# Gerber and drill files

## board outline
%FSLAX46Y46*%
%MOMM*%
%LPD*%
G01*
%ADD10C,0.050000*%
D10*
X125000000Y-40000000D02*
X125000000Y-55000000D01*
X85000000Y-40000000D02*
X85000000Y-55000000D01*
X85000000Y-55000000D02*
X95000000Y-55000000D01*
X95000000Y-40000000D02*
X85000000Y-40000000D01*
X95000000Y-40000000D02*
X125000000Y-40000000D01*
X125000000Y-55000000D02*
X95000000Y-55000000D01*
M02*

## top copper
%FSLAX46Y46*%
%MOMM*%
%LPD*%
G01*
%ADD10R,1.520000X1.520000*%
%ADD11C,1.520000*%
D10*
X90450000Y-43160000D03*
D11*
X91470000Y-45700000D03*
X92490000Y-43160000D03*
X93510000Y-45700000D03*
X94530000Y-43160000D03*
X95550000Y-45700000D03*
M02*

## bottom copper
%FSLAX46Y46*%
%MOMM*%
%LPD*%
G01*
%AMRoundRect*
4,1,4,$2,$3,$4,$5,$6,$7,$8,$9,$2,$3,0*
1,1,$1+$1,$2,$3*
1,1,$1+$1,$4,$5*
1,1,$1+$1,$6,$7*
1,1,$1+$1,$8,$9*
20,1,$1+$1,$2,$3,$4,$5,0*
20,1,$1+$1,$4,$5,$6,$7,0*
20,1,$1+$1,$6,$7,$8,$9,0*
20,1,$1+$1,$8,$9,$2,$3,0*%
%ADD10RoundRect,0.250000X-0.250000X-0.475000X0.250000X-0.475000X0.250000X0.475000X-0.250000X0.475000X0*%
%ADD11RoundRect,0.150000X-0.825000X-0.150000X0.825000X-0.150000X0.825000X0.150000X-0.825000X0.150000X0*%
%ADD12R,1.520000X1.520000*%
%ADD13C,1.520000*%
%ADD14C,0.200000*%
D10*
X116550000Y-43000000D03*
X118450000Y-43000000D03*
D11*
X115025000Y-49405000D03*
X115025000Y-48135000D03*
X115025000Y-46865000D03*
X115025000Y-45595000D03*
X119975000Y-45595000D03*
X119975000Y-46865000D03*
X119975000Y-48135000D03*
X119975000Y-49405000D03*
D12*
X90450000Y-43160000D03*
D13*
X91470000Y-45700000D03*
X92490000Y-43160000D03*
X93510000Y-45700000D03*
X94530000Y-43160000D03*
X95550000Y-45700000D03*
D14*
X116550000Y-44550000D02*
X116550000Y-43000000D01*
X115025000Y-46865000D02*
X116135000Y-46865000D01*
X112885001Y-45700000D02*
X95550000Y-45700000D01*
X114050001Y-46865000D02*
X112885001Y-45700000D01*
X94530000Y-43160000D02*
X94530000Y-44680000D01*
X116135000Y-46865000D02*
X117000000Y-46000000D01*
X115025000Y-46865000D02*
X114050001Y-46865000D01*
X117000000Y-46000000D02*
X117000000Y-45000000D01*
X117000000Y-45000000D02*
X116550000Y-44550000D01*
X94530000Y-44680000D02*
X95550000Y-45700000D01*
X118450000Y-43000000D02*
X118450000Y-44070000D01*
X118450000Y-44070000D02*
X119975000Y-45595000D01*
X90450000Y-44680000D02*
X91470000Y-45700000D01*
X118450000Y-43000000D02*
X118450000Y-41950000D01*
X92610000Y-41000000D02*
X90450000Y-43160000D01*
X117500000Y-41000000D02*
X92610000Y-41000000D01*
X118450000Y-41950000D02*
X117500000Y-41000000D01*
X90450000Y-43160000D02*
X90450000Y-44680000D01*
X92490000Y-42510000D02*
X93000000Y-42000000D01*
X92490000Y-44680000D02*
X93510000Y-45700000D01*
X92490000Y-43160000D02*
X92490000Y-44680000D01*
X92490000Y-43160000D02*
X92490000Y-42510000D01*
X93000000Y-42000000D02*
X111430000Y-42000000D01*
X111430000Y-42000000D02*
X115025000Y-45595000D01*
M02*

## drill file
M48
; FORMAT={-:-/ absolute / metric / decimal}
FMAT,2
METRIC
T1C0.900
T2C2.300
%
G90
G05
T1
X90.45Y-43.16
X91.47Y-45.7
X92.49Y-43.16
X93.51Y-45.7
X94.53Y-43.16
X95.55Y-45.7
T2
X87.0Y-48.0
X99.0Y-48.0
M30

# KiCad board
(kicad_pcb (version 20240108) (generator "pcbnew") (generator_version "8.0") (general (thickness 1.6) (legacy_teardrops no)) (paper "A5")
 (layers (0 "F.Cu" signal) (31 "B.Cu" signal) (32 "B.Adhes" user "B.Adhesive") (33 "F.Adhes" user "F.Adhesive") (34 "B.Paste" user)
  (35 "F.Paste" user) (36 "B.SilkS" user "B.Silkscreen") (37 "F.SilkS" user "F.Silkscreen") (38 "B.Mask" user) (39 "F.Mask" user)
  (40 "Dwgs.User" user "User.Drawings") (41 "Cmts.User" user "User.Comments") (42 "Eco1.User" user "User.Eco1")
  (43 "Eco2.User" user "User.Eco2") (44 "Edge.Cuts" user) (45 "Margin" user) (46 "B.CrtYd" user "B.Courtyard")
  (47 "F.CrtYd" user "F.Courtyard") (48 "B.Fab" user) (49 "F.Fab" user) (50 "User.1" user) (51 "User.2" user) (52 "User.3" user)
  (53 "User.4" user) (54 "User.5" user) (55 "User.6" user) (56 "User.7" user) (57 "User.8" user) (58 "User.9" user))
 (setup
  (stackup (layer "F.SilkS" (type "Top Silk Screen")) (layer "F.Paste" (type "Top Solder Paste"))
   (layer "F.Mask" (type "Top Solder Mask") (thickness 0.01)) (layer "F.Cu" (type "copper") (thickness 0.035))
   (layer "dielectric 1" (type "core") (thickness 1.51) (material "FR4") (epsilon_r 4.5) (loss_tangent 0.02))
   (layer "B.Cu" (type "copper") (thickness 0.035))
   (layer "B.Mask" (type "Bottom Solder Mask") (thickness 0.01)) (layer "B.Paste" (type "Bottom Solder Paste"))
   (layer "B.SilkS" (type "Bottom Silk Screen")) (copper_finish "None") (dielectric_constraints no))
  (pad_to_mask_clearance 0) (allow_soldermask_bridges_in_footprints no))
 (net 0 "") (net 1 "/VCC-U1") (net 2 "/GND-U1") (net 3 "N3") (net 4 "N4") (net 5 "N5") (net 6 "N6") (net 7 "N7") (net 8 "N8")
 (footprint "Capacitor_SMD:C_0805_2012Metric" (layer "B.Cu") (at 117.5 43)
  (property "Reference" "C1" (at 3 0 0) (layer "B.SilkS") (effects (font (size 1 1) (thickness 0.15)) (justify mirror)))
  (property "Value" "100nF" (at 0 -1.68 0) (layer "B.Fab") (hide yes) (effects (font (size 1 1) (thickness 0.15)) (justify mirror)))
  (pad "1" smd roundrect (at -0.95 0) (size 1 1.45) (layers "B.Cu" "B.Paste" "B.Mask") (roundrect_rratio 0.25) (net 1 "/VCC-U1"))
  (pad "2" smd roundrect (at 0.95 0) (size 1 1.45) (layers "B.Cu" "B.Paste" "B.Mask") (roundrect_rratio 0.25) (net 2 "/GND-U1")))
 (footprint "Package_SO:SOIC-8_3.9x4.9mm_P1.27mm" (layer "B.Cu") (at 117.5 47.5)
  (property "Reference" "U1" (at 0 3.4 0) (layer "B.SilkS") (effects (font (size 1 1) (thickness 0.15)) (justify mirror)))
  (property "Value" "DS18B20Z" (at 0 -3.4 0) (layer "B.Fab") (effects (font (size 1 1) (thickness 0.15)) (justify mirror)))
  (pad "1" smd roundrect (at -2.475 1.905) (size 1.95 0.6) (layers "B.Cu" "B.Paste" "B.Mask") (roundrect_rratio 0.25) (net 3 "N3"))
  (pad "2" smd roundrect (at -2.475 0.635) (size 1.95 0.6) (layers "B.Cu" "B.Paste" "B.Mask") (roundrect_rratio 0.25) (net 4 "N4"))
  (pad "3" smd roundrect (at -2.475 -0.635) (size 1.95 0.6) (layers "B.Cu" "B.Paste" "B.Mask") (roundrect_rratio 0.25) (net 1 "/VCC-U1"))
  (pad "4" smd roundrect (at -2.475 -1.905) (size 1.95 0.6) (layers "B.Cu" "B.Paste" "B.Mask") (roundrect_rratio 0.25) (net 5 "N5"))
  (pad "5" smd roundrect (at 2.475 -1.905) (size 1.95 0.6) (layers "B.Cu" "B.Paste" "B.Mask") (roundrect_rratio 0.25) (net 2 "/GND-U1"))
  (pad "6" smd roundrect (at 2.475 -0.635) (size 1.95 0.6) (layers "B.Cu" "B.Paste" "B.Mask") (roundrect_rratio 0.25) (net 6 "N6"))
  (pad "7" smd roundrect (at 2.475 0.635) (size 1.95 0.6) (layers "B.Cu" "B.Paste" "B.Mask") (roundrect_rratio 0.25) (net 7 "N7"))
  (pad "8" smd roundrect (at 2.475 1.905) (size 1.95 0.6) (layers "B.Cu" "B.Paste" "B.Mask") (roundrect_rratio 0.25) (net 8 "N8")))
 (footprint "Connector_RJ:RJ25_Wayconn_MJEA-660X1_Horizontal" (layer "B.Cu") (at 90.45 43.16 180)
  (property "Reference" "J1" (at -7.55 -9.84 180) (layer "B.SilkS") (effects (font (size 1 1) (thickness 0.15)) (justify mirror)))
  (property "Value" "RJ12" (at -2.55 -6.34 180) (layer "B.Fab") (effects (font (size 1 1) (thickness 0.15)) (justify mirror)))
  (pad "" np_thru_hole circle (at -8.55 -4.84 180) (size 2.3 2.3) (drill 2.3) (layers "*.Cu" "*.Mask"))
  (pad "" np_thru_hole circle (at 3.45 -4.84 180) (size 2.3 2.3) (drill 2.3) (layers "*.Cu" "*.Mask"))
  (pad "1" thru_hole rect (at 0 0 180) (size 1.52 1.52) (drill 0.9) (layers "*.Cu" "*.Mask") (remove_unused_layers no) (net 2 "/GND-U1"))
  (pad "2" thru_hole circle (at -1.02 -2.54 180) (size 1.52 1.52) (drill 0.9) (layers "*.Cu" "*.Mask") (remove_unused_layers no)
   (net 2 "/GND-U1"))
  (pad "3" thru_hole circle (at -2.04 0 180) (size 1.52 1.52) (drill 0.9) (layers "*.Cu" "*.Mask") (remove_unused_layers no) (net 5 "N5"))
  (pad "4" thru_hole circle (at -3.06 -2.54 180) (size 1.52 1.52) (drill 0.9) (layers "*.Cu" "*.Mask") (remove_unused_layers no)
   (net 5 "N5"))
  (pad "5" thru_hole circle (at -4.08 0 180) (size 1.52 1.52) (drill 0.9) (layers "*.Cu" "*.Mask") (remove_unused_layers no)
   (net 1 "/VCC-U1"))
  (pad "6" thru_hole circle (at -5.1 -2.54 180) (size 1.52 1.52) (drill 0.9) (layers "*.Cu" "*.Mask") (remove_unused_layers no)
   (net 1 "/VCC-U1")))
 (gr_line (start 125 40) (end 125 55) (stroke (width 0.05) (type default)) (layer "Edge.Cuts"))
 (gr_line (start 85 40) (end 85 55) (stroke (width 0.05) (type default)) (layer "Edge.Cuts"))
 (gr_line (start 85 55) (end 95 55) (stroke (width 0.05) (type default)) (layer "Edge.Cuts"))
 (gr_line (start 95 40) (end 85 40) (stroke (width 0.05) (type default)) (layer "Edge.Cuts"))
 (gr_line (start 95 40) (end 125 40) (stroke (width 0.05) (type default)) (layer "Edge.Cuts"))
 (gr_line (start 125 55) (end 95 55) (stroke (width 0.05) (type default)) (layer "Edge.Cuts"))
 (segment (start 116.55 44.55) (end 116.55 43) (width 0.2) (layer "B.Cu") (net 1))
 (segment (start 115.025 46.865) (end 116.135 46.865) (width 0.2) (layer "B.Cu") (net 1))
 (segment (start 112.885001 45.7) (end 95.55 45.7) (width 0.2) (layer "B.Cu") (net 1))
 (segment (start 114.050001 46.865) (end 112.885001 45.7) (width 0.2) (layer "B.Cu") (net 1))
 (segment (start 94.53 43.16) (end 94.53 44.68) (width 0.2) (layer "B.Cu") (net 1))
 (segment (start 116.135 46.865) (end 117 46) (width 0.2) (layer "B.Cu") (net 1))
 (segment (start 115.025 46.865) (end 114.050001 46.865) (width 0.2) (layer "B.Cu") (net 1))
 (segment (start 117 46) (end 117 45) (width 0.2) (layer "B.Cu") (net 1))
 (segment (start 117 45) (end 116.55 44.55) (width 0.2) (layer "B.Cu") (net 1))
 (segment (start 94.53 44.68) (end 95.55 45.7) (width 0.2) (layer "B.Cu") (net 1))
 (segment (start 118.45 43) (end 118.45 44.07) (width 0.2) (layer "B.Cu") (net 2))
 (segment (start 118.45 44.07) (end 119.975 45.595) (width 0.2) (layer "B.Cu") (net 2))
 (segment (start 90.45 44.68) (end 91.47 45.7) (width 0.2) (layer "B.Cu") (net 2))
 (segment (start 118.45 43) (end 118.45 41.95) (width 0.2) (layer "B.Cu") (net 2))
 (segment (start 92.61 41) (end 90.45 43.16) (width 0.2) (layer "B.Cu") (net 2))
 (segment (start 117.5 41) (end 92.61 41) (width 0.2) (layer "B.Cu") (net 2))
 (segment (start 118.45 41.95) (end 117.5 41) (width 0.2) (layer "B.Cu") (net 2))
 (segment (start 90.45 43.16) (end 90.45 44.68) (width 0.2) (layer "B.Cu") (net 2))
 (segment (start 92.49 42.51) (end 93 42) (width 0.2) (layer "B.Cu") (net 5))
 (segment (start 92.49 44.68) (end 93.51 45.7) (width 0.2) (layer "B.Cu") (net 5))
 (segment (start 92.49 43.16) (end 92.49 44.68) (width 0.2) (layer "B.Cu") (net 5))
 (segment (start 92.49 43.16) (end 92.49 42.51) (width 0.2) (layer "B.Cu") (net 5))
 (segment (start 93 42) (end 111.43 42) (width 0.2) (layer "B.Cu") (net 5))
 (segment (start 111.43 42) (end 115.025 45.595) (width 0.2) (layer "B.Cu") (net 5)))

